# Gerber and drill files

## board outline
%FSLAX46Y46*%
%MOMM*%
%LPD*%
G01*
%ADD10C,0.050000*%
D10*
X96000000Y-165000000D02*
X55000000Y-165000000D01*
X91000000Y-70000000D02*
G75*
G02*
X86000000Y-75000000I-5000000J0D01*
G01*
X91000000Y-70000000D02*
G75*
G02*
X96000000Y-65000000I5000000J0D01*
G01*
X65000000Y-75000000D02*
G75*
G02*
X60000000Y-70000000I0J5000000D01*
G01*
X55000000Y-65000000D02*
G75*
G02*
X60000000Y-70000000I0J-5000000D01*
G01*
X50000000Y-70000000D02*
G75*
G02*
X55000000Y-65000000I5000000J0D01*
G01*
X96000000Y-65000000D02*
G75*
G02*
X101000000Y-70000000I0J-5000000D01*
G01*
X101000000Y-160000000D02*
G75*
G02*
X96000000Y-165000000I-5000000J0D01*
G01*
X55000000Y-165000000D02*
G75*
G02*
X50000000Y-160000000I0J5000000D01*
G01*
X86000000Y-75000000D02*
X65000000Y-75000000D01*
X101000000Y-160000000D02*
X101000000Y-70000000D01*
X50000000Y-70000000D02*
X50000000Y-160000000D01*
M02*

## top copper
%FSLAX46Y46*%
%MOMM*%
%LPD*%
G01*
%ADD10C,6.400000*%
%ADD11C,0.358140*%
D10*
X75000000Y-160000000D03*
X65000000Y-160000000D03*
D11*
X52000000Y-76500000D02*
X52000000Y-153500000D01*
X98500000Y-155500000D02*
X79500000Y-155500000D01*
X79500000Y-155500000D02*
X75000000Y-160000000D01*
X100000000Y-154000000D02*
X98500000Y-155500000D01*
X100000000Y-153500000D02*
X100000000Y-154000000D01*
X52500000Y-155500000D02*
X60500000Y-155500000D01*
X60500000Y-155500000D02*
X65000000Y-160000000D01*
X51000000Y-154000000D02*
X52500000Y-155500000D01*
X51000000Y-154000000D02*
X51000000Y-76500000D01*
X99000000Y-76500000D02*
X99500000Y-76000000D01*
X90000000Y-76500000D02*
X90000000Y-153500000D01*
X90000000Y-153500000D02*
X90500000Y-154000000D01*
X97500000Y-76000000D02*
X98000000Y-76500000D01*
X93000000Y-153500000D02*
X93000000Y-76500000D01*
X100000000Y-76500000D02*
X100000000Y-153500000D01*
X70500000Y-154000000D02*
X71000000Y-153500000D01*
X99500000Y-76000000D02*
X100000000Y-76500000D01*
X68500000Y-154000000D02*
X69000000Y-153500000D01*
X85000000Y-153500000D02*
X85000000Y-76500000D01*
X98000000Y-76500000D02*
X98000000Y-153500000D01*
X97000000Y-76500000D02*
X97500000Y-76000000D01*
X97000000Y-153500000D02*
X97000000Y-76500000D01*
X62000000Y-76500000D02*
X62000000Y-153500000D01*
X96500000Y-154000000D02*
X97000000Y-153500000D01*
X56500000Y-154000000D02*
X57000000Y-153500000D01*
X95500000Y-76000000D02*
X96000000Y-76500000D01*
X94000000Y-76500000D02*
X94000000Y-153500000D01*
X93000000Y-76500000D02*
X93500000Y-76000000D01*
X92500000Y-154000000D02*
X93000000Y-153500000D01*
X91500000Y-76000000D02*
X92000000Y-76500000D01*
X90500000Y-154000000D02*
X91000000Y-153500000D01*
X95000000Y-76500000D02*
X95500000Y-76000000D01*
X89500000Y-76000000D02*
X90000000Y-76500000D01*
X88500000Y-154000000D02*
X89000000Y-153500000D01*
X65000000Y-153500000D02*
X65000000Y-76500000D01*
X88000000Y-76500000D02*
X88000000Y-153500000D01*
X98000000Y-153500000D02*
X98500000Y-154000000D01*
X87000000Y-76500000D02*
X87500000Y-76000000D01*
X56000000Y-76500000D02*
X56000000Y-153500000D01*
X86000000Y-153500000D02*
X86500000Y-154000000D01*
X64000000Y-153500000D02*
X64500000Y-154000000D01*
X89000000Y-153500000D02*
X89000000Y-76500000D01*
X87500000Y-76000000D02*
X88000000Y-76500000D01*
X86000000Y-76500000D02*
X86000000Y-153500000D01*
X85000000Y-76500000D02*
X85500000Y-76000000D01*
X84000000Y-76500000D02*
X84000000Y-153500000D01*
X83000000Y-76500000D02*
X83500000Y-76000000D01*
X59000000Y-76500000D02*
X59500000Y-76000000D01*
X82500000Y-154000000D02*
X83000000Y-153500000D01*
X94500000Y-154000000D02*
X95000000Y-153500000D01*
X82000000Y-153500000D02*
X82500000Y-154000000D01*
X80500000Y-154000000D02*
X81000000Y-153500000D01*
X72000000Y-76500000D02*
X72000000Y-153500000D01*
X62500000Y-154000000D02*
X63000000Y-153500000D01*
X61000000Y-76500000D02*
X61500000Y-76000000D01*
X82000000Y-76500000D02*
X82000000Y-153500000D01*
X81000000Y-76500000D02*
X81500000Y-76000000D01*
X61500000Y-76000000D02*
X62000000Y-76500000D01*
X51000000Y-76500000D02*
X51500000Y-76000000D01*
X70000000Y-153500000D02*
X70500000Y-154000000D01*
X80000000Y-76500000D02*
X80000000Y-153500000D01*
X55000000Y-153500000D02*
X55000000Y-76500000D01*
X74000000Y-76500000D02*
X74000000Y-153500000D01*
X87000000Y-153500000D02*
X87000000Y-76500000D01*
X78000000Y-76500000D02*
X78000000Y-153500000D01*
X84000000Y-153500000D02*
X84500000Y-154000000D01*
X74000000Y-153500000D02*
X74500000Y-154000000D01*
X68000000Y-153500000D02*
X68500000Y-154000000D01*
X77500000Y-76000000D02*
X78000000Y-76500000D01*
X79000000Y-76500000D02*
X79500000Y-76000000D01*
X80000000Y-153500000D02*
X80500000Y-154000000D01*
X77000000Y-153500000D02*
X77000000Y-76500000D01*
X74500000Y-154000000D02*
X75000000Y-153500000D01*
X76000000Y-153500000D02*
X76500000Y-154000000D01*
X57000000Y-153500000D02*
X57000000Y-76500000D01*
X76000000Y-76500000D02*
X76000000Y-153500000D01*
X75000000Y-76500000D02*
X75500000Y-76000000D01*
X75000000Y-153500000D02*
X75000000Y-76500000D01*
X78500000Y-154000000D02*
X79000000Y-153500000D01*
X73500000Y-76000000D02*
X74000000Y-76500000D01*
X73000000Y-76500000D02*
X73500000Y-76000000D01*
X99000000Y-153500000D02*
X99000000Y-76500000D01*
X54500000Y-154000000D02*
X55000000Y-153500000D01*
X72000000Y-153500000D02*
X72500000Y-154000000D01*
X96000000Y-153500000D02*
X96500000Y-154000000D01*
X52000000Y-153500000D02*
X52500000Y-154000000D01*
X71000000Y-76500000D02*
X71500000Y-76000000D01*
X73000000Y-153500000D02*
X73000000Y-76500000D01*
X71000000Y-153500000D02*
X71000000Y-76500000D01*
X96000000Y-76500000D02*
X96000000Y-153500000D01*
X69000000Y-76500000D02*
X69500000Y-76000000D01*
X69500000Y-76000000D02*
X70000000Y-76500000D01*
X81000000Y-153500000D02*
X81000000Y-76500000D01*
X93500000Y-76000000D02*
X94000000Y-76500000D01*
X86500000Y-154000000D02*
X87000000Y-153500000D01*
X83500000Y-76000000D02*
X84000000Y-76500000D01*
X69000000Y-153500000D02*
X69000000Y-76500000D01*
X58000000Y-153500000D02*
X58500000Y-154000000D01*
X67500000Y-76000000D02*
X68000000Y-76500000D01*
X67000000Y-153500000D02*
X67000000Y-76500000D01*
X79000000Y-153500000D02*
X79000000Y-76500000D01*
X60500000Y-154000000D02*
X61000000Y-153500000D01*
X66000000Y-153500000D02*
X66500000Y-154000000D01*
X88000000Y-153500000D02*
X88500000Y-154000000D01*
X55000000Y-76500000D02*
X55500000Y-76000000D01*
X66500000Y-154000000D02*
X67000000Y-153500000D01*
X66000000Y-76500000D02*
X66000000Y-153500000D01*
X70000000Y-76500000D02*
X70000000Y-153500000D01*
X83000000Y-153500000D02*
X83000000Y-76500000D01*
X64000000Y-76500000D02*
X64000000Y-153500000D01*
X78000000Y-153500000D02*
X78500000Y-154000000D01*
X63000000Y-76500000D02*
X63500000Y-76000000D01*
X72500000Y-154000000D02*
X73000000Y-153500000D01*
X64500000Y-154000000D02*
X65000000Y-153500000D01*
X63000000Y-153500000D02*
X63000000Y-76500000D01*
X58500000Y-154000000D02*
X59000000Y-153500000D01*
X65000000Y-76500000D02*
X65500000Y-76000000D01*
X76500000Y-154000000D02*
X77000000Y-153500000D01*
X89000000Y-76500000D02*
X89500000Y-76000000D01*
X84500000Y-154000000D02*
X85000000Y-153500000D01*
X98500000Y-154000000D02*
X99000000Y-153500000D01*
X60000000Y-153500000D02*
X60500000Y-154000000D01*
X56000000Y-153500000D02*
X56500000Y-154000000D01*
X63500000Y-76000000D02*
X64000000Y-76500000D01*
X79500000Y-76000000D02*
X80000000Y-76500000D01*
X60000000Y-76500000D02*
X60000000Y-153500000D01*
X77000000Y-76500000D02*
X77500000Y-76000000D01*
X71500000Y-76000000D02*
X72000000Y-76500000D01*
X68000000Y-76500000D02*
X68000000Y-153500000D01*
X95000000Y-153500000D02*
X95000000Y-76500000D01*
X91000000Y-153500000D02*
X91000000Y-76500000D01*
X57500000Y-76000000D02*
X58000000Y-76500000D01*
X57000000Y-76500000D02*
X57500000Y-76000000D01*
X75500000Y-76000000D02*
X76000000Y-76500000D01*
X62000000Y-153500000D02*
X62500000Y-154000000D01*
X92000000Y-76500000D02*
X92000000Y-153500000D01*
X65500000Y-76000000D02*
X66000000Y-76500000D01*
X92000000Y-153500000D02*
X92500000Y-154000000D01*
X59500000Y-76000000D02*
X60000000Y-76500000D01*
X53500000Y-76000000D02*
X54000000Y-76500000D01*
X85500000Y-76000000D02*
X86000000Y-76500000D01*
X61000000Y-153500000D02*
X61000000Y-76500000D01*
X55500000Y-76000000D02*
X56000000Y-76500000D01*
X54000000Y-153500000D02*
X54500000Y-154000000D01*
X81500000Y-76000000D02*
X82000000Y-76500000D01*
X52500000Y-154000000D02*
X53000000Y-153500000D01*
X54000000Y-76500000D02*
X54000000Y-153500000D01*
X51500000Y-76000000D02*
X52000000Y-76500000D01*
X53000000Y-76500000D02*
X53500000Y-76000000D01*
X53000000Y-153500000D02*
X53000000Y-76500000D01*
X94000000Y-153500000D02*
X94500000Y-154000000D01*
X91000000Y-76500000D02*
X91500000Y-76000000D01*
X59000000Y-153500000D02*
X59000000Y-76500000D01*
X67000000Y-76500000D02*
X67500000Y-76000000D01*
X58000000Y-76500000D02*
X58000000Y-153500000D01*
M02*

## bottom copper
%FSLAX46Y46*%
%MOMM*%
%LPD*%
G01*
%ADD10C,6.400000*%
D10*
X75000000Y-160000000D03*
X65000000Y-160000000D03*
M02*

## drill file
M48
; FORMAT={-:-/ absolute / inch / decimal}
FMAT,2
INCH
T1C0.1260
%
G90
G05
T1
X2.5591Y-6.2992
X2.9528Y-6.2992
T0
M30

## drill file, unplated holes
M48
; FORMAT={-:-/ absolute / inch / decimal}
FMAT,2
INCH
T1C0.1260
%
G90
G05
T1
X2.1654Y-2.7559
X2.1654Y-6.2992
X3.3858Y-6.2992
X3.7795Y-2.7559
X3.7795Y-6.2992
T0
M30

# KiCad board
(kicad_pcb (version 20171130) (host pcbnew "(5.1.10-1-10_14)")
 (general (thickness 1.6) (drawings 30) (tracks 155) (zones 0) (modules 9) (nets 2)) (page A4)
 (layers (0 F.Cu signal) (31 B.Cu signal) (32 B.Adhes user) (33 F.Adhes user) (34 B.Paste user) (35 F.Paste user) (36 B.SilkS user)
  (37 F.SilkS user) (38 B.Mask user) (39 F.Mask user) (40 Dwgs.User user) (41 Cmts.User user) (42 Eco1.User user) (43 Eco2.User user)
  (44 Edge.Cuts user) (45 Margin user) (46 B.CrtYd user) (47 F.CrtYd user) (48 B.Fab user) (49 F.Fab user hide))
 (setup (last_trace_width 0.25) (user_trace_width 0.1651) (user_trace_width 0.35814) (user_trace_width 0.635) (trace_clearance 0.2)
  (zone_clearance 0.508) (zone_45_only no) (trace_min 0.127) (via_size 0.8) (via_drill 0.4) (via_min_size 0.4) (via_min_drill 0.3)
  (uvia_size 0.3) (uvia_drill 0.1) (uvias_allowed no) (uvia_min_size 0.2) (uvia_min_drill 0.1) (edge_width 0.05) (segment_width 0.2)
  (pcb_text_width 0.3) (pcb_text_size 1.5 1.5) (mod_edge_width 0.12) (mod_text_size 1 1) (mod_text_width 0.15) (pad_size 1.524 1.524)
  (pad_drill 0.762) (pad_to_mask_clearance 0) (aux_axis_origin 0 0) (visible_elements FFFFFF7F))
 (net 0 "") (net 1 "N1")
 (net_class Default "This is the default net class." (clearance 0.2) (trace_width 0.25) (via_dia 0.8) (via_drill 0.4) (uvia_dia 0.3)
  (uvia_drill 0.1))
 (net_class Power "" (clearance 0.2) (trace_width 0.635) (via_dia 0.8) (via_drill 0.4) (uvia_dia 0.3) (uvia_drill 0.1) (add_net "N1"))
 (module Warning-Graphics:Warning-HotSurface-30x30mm (layer B.Cu) (at 75.6666 105.6132)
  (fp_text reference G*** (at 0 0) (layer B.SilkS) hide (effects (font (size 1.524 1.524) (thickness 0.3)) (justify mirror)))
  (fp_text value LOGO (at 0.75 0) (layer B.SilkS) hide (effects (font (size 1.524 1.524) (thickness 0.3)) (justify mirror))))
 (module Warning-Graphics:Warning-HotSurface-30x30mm (layer F.Cu) (at 75.4888 122.8852)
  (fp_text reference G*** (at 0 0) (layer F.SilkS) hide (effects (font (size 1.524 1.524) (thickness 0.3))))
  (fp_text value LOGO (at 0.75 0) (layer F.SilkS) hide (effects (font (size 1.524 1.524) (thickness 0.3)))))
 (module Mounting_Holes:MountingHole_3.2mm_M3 (layer F.Cu) (at 86 160)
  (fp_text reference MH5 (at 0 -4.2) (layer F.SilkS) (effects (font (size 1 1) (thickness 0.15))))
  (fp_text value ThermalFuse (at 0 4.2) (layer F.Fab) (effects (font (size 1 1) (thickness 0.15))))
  (pad 1 np_thru_hole circle (at 0 0) (size 3.2 3.2) (drill 3.2) (layers *.Cu *.Mask)))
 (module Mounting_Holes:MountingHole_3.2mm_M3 (layer F.Cu) (at 96 160)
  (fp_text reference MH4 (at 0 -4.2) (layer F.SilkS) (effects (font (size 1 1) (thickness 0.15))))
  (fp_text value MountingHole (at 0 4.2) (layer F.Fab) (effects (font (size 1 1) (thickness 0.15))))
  (pad 1 np_thru_hole circle (at 0 0) (size 3.2 3.2) (drill 3.2) (layers *.Cu *.Mask)))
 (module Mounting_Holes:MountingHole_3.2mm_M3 (layer F.Cu) (at 96 70)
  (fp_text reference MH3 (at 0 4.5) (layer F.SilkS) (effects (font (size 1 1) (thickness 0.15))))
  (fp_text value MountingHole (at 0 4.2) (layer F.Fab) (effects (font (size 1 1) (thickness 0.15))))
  (pad 1 np_thru_hole circle (at 0 0) (size 3.2 3.2) (drill 3.2) (layers *.Cu *.Mask)))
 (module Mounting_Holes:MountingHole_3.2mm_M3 (layer F.Cu) (at 55 70)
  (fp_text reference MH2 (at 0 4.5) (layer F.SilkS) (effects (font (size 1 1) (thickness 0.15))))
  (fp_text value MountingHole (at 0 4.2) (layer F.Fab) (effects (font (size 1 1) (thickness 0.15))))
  (pad 1 np_thru_hole circle (at 0 0) (size 3.2 3.2) (drill 3.2) (layers *.Cu *.Mask)))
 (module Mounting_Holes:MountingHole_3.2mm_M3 (layer F.Cu) (at 55 160)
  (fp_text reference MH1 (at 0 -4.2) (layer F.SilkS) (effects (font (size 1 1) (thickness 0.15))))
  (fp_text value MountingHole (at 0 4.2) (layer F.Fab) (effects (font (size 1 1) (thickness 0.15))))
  (pad 1 np_thru_hole circle (at 0 0) (size 3.2 3.2) (drill 3.2) (layers *.Cu *.Mask)))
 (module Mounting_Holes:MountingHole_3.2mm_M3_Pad (layer F.Cu) (at 75 160)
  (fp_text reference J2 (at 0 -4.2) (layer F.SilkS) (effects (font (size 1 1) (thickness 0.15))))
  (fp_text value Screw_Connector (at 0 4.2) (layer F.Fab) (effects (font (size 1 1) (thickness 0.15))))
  (pad 1 thru_hole circle (at 0 0) (size 6.4 6.4) (drill 3.2) (layers *.Cu *.Mask) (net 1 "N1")))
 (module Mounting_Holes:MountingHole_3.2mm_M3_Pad (layer F.Cu) (at 65 160)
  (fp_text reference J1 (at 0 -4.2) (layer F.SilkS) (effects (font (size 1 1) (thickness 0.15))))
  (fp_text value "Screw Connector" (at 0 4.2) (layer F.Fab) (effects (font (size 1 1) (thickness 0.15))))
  (pad 1 thru_hole circle (at 0 0) (size 6.4 6.4) (drill 3.2) (layers *.Cu *.Mask) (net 1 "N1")))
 (gr_line (start 96 165) (end 55 165) (layer Edge.Cuts) (width 0.05))
 (gr_arc (start 86 70) (end 86 75) (angle -90) (layer Edge.Cuts) (width 0.05))
 (gr_arc (start 96 70) (end 96 65) (angle -90) (layer Edge.Cuts) (width 0.05))
 (gr_arc (start 65 70) (end 60 70) (angle -90) (layer Edge.Cuts) (width 0.05))
 (gr_arc (start 55 70) (end 60 70) (angle -90) (layer Edge.Cuts) (width 0.05))
 (gr_arc (start 55 70) (end 55 65) (angle -90) (layer Edge.Cuts) (width 0.05))
 (gr_arc (start 96 70) (end 101 70) (angle -90) (layer Edge.Cuts) (width 0.05))
 (gr_arc (start 96 160) (end 96 165) (angle -90) (layer Edge.Cuts) (width 0.05))
 (gr_arc (start 55 160) (end 50 160) (angle -90) (layer Edge.Cuts) (width 0.05))
 (gr_line (start 86 75) (end 65 75) (layer Edge.Cuts) (width 0.05))
 (gr_line (start 101 160) (end 101 70) (layer Edge.Cuts) (width 0.05))
 (gr_line (start 50 70) (end 50 160) (layer Edge.Cuts) (width 0.05))
 (segment (start 52 76.5) (end 52 153.5) (width 0.35814) (layer F.Cu) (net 1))
 (segment (start 98.5 155.5) (end 79.5 155.5) (width 0.35814) (layer F.Cu) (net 1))
 (segment (start 79.5 155.5) (end 75 160) (width 0.35814) (layer F.Cu) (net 1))
 (segment (start 100 154) (end 98.5 155.5) (width 0.35814) (layer F.Cu) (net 1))
 (segment (start 100 153.5) (end 100 154) (width 0.35814) (layer F.Cu) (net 1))
 (segment (start 52.5 155.5) (end 60.5 155.5) (width 0.35814) (layer F.Cu) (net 1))
 (segment (start 60.5 155.5) (end 65 160) (width 0.35814) (layer F.Cu) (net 1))
 (segment (start 51 154) (end 52.5 155.5) (width 0.35814) (layer F.Cu) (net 1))
 (segment (start 51 154) (end 51 76.5) (width 0.35814) (layer F.Cu) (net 1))
 (segment (start 99 76.5) (end 99.5 76) (width 0.35814) (layer F.Cu) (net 1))
 (segment (start 90 76.5) (end 90 153.5) (width 0.35814) (layer F.Cu) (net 1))
 (segment (start 90 153.5) (end 90.5 154) (width 0.35814) (layer F.Cu) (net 1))
 (segment (start 97.5 76) (end 98 76.5) (width 0.35814) (layer F.Cu) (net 1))
 (segment (start 93 153.5) (end 93 76.5) (width 0.35814) (layer F.Cu) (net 1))
 (segment (start 100 76.5) (end 100 153.5) (width 0.35814) (layer F.Cu) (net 1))
 (segment (start 70.5 154) (end 71 153.5) (width 0.35814) (layer F.Cu) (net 1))
 (segment (start 99.5 76) (end 100 76.5) (width 0.35814) (layer F.Cu) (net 1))
 (segment (start 68.5 154) (end 69 153.5) (width 0.35814) (layer F.Cu) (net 1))
 (segment (start 85 153.5) (end 85 76.5) (width 0.35814) (layer F.Cu) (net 1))
 (segment (start 98 76.5) (end 98 153.5) (width 0.35814) (layer F.Cu) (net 1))
 (segment (start 97 76.5) (end 97.5 76) (width 0.35814) (layer F.Cu) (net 1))
 (segment (start 97 153.5) (end 97 76.5) (width 0.35814) (layer F.Cu) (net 1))
 (segment (start 62 76.5) (end 62 153.5) (width 0.35814) (layer F.Cu) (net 1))
 (segment (start 96.5 154) (end 97 153.5) (width 0.35814) (layer F.Cu) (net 1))
 (segment (start 56.5 154) (end 57 153.5) (width 0.35814) (layer F.Cu) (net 1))
 (segment (start 95.5 76) (end 96 76.5) (width 0.35814) (layer F.Cu) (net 1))
 (segment (start 94 76.5) (end 94 153.5) (width 0.35814) (layer F.Cu) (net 1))
 (segment (start 93 76.5) (end 93.5 76) (width 0.35814) (layer F.Cu) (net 1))
 (segment (start 92.5 154) (end 93 153.5) (width 0.35814) (layer F.Cu) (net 1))
 (segment (start 91.5 76) (end 92 76.5) (width 0.35814) (layer F.Cu) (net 1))
 (segment (start 90.5 154) (end 91 153.5) (width 0.35814) (layer F.Cu) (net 1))
 (segment (start 95 76.5) (end 95.5 76) (width 0.35814) (layer F.Cu) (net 1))
 (segment (start 89.5 76) (end 90 76.5) (width 0.35814) (layer F.Cu) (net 1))
 (segment (start 88.5 154) (end 89 153.5) (width 0.35814) (layer F.Cu) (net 1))
 (segment (start 65 153.5) (end 65 76.5) (width 0.35814) (layer F.Cu) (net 1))
 (segment (start 88 76.5) (end 88 153.5) (width 0.35814) (layer F.Cu) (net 1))
 (segment (start 98 153.5) (end 98.5 154) (width 0.35814) (layer F.Cu) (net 1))
 (segment (start 87 76.5) (end 87.5 76) (width 0.35814) (layer F.Cu) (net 1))
 (segment (start 56 76.5) (end 56 153.5) (width 0.35814) (layer F.Cu) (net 1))
 (segment (start 86 153.5) (end 86.5 154) (width 0.35814) (layer F.Cu) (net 1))
 (segment (start 64 153.5) (end 64.5 154) (width 0.35814) (layer F.Cu) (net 1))
 (segment (start 89 153.5) (end 89 76.5) (width 0.35814) (layer F.Cu) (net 1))
 (segment (start 87.5 76) (end 88 76.5) (width 0.35814) (layer F.Cu) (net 1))
 (segment (start 86 76.5) (end 86 153.5) (width 0.35814) (layer F.Cu) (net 1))
 (segment (start 85 76.5) (end 85.5 76) (width 0.35814) (layer F.Cu) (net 1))
 (segment (start 84 76.5) (end 84 153.5) (width 0.35814) (layer F.Cu) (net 1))
 (segment (start 83 76.5) (end 83.5 76) (width 0.35814) (layer F.Cu) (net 1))
 (segment (start 59 76.5) (end 59.5 76) (width 0.35814) (layer F.Cu) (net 1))
 (segment (start 82.5 154) (end 83 153.5) (width 0.35814) (layer F.Cu) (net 1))
 (segment (start 94.5 154) (end 95 153.5) (width 0.35814) (layer F.Cu) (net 1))
 (segment (start 82 153.5) (end 82.5 154) (width 0.35814) (layer F.Cu) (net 1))
 (segment (start 80.5 154) (end 81 153.5) (width 0.35814) (layer F.Cu) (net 1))
 (segment (start 72 76.5) (end 72 153.5) (width 0.35814) (layer F.Cu) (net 1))
 (segment (start 62.5 154) (end 63 153.5) (width 0.35814) (layer F.Cu) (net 1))
 (segment (start 61 76.5) (end 61.5 76) (width 0.35814) (layer F.Cu) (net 1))
 (segment (start 82 76.5) (end 82 153.5) (width 0.35814) (layer F.Cu) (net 1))
 (segment (start 81 76.5) (end 81.5 76) (width 0.35814) (layer F.Cu) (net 1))
 (segment (start 61.5 76) (end 62 76.5) (width 0.35814) (layer F.Cu) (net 1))
 (segment (start 51 76.5) (end 51.5 76) (width 0.35814) (layer F.Cu) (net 1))
 (segment (start 70 153.5) (end 70.5 154) (width 0.35814) (layer F.Cu) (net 1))
 (segment (start 80 76.5) (end 80 153.5) (width 0.35814) (layer F.Cu) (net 1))
 (segment (start 55 153.5) (end 55 76.5) (width 0.35814) (layer F.Cu) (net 1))
 (segment (start 74 76.5) (end 74 153.5) (width 0.35814) (layer F.Cu) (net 1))
 (segment (start 87 153.5) (end 87 76.5) (width 0.35814) (layer F.Cu) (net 1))
 (segment (start 78 76.5) (end 78 153.5) (width 0.35814) (layer F.Cu) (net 1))
 (segment (start 84 153.5) (end 84.5 154) (width 0.35814) (layer F.Cu) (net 1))
 (segment (start 74 153.5) (end 74.5 154) (width 0.35814) (layer F.Cu) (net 1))
 (segment (start 68 153.5) (end 68.5 154) (width 0.35814) (layer F.Cu) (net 1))
 (segment (start 77.5 76) (end 78 76.5) (width 0.35814) (layer F.Cu) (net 1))
 (segment (start 79 76.5) (end 79.5 76) (width 0.35814) (layer F.Cu) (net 1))
 (segment (start 80 153.5) (end 80.5 154) (width 0.35814) (layer F.Cu) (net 1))
 (segment (start 77 153.5) (end 77 76.5) (width 0.35814) (layer F.Cu) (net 1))
 (segment (start 74.5 154) (end 75 153.5) (width 0.35814) (layer F.Cu) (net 1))
 (segment (start 76 153.5) (end 76.5 154) (width 0.35814) (layer F.Cu) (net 1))
 (segment (start 57 153.5) (end 57 76.5) (width 0.35814) (layer F.Cu) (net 1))
 (segment (start 76 76.5) (end 76 153.5) (width 0.35814) (layer F.Cu) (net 1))
 (segment (start 75 76.5) (end 75.5 76) (width 0.35814) (layer F.Cu) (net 1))
 (segment (start 75 153.5) (end 75 76.5) (width 0.35814) (layer F.Cu) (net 1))
 (segment (start 78.5 154) (end 79 153.5) (width 0.35814) (layer F.Cu) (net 1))
 (segment (start 73.5 76) (end 74 76.5) (width 0.35814) (layer F.Cu) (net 1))
 (segment (start 73 76.5) (end 73.5 76) (width 0.35814) (layer F.Cu) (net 1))
 (segment (start 99 153.5) (end 99 76.5) (width 0.35814) (layer F.Cu) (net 1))
 (segment (start 54.5 154) (end 55 153.5) (width 0.35814) (layer F.Cu) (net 1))
 (segment (start 72 153.5) (end 72.5 154) (width 0.35814) (layer F.Cu) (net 1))
 (segment (start 96 153.5) (end 96.5 154) (width 0.35814) (layer F.Cu) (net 1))
 (segment (start 52 153.5) (end 52.5 154) (width 0.35814) (layer F.Cu) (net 1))
 (segment (start 71 76.5) (end 71.5 76) (width 0.35814) (layer F.Cu) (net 1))
 (segment (start 73 153.5) (end 73 76.5) (width 0.35814) (layer F.Cu) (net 1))
 (segment (start 71 153.5) (end 71 76.5) (width 0.35814) (layer F.Cu) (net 1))
 (segment (start 96 76.5) (end 96 153.5) (width 0.35814) (layer F.Cu) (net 1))
 (segment (start 69 76.5) (end 69.5 76) (width 0.35814) (layer F.Cu) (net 1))
 (segment (start 69.5 76) (end 70 76.5) (width 0.35814) (layer F.Cu) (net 1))
 (segment (start 81 153.5) (end 81 76.5) (width 0.35814) (layer F.Cu) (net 1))
 (segment (start 93.5 76) (end 94 76.5) (width 0.35814) (layer F.Cu) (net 1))
 (segment (start 86.5 154) (end 87 153.5) (width 0.35814) (layer F.Cu) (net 1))
 (segment (start 83.5 76) (end 84 76.5) (width 0.35814) (layer F.Cu) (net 1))
 (segment (start 69 153.5) (end 69 76.5) (width 0.35814) (layer F.Cu) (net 1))
 (segment (start 58 153.5) (end 58.5 154) (width 0.35814) (layer F.Cu) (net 1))
 (segment (start 67.5 76) (end 68 76.5) (width 0.35814) (layer F.Cu) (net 1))
 (segment (start 67 153.5) (end 67 76.5) (width 0.35814) (layer F.Cu) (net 1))
 (segment (start 79 153.5) (end 79 76.5) (width 0.35814) (layer F.Cu) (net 1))
 (segment (start 60.5 154) (end 61 153.5) (width 0.35814) (layer F.Cu) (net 1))
 (segment (start 66 153.5) (end 66.5 154) (width 0.35814) (layer F.Cu) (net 1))
 (segment (start 88 153.5) (end 88.5 154) (width 0.35814) (layer F.Cu) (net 1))
 (segment (start 55 76.5) (end 55.5 76) (width 0.35814) (layer F.Cu) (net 1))
 (segment (start 66.5 154) (end 67 153.5) (width 0.35814) (layer F.Cu) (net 1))
 (segment (start 66 76.5) (end 66 153.5) (width 0.35814) (layer F.Cu) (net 1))
 (segment (start 70 76.5) (end 70 153.5) (width 0.35814) (layer F.Cu) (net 1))
 (segment (start 83 153.5) (end 83 76.5) (width 0.35814) (layer F.Cu) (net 1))
 (segment (start 64 76.5) (end 64 153.5) (width 0.35814) (layer F.Cu) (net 1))
 (segment (start 78 153.5) (end 78.5 154) (width 0.35814) (layer F.Cu) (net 1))
 (segment (start 63 76.5) (end 63.5 76) (width 0.35814) (layer F.Cu) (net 1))
 (segment (start 72.5 154) (end 73 153.5) (width 0.35814) (layer F.Cu) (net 1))
 (segment (start 64.5 154) (end 65 153.5) (width 0.35814) (layer F.Cu) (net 1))
 (segment (start 63 153.5) (end 63 76.5) (width 0.35814) (layer F.Cu) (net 1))
 (segment (start 58.5 154) (end 59 153.5) (width 0.35814) (layer F.Cu) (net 1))
 (segment (start 65 76.5) (end 65.5 76) (width 0.35814) (layer F.Cu) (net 1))
 (segment (start 76.5 154) (end 77 153.5) (width 0.35814) (layer F.Cu) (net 1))
 (segment (start 89 76.5) (end 89.5 76) (width 0.35814) (layer F.Cu) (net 1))
 (segment (start 84.5 154) (end 85 153.5) (width 0.35814) (layer F.Cu) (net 1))
 (segment (start 98.5 154) (end 99 153.5) (width 0.35814) (layer F.Cu) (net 1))
 (segment (start 60 153.5) (end 60.5 154) (width 0.35814) (layer F.Cu) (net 1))
 (segment (start 56 153.5) (end 56.5 154) (width 0.35814) (layer F.Cu) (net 1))
 (segment (start 63.5 76) (end 64 76.5) (width 0.35814) (layer F.Cu) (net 1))
 (segment (start 79.5 76) (end 80 76.5) (width 0.35814) (layer F.Cu) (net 1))
 (segment (start 60 76.5) (end 60 153.5) (width 0.35814) (layer F.Cu) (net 1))
 (segment (start 77 76.5) (end 77.5 76) (width 0.35814) (layer F.Cu) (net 1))
 (segment (start 71.5 76) (end 72 76.5) (width 0.35814) (layer F.Cu) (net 1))
 (segment (start 68 76.5) (end 68 153.5) (width 0.35814) (layer F.Cu) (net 1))
 (segment (start 95 153.5) (end 95 76.5) (width 0.35814) (layer F.Cu) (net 1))
 (segment (start 91 153.5) (end 91 76.5) (width 0.35814) (layer F.Cu) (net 1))
 (segment (start 57.5 76) (end 58 76.5) (width 0.35814) (layer F.Cu) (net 1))
 (segment (start 57 76.5) (end 57.5 76) (width 0.35814) (layer F.Cu) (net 1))
 (segment (start 75.5 76) (end 76 76.5) (width 0.35814) (layer F.Cu) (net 1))
 (segment (start 62 153.5) (end 62.5 154) (width 0.35814) (layer F.Cu) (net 1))
 (segment (start 92 76.5) (end 92 153.5) (width 0.35814) (layer F.Cu) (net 1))
 (segment (start 65.5 76) (end 66 76.5) (width 0.35814) (layer F.Cu) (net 1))
 (segment (start 92 153.5) (end 92.5 154) (width 0.35814) (layer F.Cu) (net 1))
 (segment (start 59.5 76) (end 60 76.5) (width 0.35814) (layer F.Cu) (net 1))
 (segment (start 53.5 76) (end 54 76.5) (width 0.35814) (layer F.Cu) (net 1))
 (segment (start 85.5 76) (end 86 76.5) (width 0.35814) (layer F.Cu) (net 1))
 (segment (start 61 153.5) (end 61 76.5) (width 0.35814) (layer F.Cu) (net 1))
 (segment (start 55.5 76) (end 56 76.5) (width 0.35814) (layer F.Cu) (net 1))
 (segment (start 54 153.5) (end 54.5 154) (width 0.35814) (layer F.Cu) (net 1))
 (segment (start 81.5 76) (end 82 76.5) (width 0.35814) (layer F.Cu) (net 1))
 (segment (start 52.5 154) (end 53 153.5) (width 0.35814) (layer F.Cu) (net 1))
 (segment (start 54 76.5) (end 54 153.5) (width 0.35814) (layer F.Cu) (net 1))
 (segment (start 51.5 76) (end 52 76.5) (width 0.35814) (layer F.Cu) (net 1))
 (segment (start 53 76.5) (end 53.5 76) (width 0.35814) (layer F.Cu) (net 1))
 (segment (start 53 153.5) (end 53 76.5) (width 0.35814) (layer F.Cu) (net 1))
 (segment (start 94 153.5) (end 94.5 154) (width 0.35814) (layer F.Cu) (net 1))
 (segment (start 91 76.5) (end 91.5 76) (width 0.35814) (layer F.Cu) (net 1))
 (segment (start 59 153.5) (end 59 76.5) (width 0.35814) (layer F.Cu) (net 1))
 (segment (start 67 76.5) (end 67.5 76) (width 0.35814) (layer F.Cu) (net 1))
 (segment (start 58 76.5) (end 58 153.5) (width 0.35814) (layer F.Cu) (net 1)))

